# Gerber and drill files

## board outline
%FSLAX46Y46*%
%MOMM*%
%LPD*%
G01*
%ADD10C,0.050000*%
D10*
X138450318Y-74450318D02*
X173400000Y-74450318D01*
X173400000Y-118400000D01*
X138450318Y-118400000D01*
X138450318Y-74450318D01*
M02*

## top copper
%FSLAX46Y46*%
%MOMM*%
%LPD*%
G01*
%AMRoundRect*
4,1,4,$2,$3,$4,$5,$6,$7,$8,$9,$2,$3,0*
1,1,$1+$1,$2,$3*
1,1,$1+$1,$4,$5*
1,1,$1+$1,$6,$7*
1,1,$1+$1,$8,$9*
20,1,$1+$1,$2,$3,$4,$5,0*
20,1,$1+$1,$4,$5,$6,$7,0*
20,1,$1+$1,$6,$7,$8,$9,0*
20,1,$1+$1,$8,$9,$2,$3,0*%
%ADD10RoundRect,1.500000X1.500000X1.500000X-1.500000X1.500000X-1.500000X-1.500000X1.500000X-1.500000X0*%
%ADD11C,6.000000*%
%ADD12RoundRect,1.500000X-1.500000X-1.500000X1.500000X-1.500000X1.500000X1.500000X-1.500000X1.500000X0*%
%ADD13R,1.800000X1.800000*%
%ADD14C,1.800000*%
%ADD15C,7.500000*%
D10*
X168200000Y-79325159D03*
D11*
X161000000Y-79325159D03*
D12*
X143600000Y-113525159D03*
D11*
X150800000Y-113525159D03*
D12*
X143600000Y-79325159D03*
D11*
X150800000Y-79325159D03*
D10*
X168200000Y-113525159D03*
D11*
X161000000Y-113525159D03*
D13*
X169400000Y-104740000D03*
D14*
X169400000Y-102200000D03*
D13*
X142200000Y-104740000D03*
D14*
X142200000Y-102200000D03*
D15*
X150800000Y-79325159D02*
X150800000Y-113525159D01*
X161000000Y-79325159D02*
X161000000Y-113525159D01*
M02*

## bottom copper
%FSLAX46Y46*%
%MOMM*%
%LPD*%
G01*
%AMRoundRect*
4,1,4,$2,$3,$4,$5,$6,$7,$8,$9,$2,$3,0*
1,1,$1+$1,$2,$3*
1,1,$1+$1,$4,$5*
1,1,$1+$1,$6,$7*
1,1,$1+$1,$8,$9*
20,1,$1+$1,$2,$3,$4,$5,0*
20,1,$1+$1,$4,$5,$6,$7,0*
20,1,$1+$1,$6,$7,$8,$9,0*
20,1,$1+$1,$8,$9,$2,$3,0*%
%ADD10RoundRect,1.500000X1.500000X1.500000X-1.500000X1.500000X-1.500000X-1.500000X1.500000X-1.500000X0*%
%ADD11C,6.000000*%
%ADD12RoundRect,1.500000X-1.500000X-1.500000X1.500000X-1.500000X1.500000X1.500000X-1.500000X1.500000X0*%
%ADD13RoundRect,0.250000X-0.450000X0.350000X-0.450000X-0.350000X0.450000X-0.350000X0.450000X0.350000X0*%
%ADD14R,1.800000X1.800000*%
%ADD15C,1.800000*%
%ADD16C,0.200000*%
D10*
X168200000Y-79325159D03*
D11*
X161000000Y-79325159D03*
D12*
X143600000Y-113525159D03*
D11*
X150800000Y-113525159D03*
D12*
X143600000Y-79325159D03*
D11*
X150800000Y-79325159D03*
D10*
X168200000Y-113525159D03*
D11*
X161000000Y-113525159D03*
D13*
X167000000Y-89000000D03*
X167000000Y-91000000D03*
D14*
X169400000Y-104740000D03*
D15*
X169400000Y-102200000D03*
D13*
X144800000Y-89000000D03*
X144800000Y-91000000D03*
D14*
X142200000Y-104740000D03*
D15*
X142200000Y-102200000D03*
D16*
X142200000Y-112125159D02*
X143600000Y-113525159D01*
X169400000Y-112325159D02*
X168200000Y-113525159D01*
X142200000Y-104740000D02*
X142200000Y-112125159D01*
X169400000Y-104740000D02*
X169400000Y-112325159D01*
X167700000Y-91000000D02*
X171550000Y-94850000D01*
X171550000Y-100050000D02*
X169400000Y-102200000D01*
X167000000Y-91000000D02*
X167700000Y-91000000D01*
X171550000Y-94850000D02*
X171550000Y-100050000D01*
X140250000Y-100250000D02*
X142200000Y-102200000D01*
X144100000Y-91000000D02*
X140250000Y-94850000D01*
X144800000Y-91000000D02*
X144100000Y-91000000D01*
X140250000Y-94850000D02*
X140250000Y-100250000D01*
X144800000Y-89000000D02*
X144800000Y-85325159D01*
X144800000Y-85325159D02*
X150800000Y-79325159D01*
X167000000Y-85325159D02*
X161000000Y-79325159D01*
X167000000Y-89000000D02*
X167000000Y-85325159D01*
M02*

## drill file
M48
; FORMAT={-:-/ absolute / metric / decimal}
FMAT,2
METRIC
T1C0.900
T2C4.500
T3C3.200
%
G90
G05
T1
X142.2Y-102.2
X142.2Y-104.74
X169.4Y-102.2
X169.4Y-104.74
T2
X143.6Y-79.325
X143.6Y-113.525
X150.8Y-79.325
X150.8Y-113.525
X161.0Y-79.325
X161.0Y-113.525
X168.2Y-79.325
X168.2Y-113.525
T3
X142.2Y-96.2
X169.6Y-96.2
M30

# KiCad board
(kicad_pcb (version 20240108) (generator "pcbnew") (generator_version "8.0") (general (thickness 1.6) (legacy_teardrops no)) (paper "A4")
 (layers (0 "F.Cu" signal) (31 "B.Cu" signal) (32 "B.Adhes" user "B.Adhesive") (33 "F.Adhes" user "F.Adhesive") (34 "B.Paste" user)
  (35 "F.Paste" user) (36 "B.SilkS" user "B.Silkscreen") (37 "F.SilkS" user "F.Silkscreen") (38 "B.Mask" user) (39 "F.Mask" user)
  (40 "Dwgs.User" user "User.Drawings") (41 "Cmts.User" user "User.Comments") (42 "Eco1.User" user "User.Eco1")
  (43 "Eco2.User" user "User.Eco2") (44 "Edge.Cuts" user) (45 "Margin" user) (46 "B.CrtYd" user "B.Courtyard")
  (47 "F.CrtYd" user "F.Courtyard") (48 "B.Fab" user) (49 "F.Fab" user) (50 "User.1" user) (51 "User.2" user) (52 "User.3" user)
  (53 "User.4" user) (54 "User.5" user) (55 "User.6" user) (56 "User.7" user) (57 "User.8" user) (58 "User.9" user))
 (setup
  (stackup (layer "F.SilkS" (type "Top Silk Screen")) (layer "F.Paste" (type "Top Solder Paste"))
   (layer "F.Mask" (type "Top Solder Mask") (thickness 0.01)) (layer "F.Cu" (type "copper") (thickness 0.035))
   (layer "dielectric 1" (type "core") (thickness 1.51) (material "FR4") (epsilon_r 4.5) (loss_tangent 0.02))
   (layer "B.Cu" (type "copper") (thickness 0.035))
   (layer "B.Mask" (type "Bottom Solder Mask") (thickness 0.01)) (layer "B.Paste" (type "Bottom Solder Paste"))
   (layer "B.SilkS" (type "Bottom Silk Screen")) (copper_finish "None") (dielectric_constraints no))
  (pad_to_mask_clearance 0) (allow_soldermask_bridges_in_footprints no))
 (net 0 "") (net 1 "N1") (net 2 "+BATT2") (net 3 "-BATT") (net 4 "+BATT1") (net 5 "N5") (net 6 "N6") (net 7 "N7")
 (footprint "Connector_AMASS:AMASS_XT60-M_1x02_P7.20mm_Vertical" (layer "F.Cu") (at 168.2 79.325159 180)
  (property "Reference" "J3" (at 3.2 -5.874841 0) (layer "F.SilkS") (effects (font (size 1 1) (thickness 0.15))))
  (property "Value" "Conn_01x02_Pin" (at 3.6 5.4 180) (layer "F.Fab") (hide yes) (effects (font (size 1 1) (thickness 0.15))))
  (pad "1" thru_hole roundrect (at 0 0 180) (size 6 6) (drill 4.5) (layers "*.Cu" "*.Mask") (remove_unused_layers no)
   (roundrect_rratio 0.25) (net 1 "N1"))
  (pad "2" thru_hole circle (at 7.2 0 180) (size 6 6) (drill 4.5) (layers "*.Cu" "*.Mask") (remove_unused_layers no) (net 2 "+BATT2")))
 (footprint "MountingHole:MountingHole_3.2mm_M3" (layer "F.Cu") (at 169.6 96.2)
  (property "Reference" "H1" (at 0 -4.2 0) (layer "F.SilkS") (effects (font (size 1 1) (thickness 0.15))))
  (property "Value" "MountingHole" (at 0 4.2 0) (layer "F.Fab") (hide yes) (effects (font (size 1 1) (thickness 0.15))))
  (pad "" np_thru_hole circle (at 0 0) (size 3.2 3.2) (drill 3.2) (layers "*.Cu" "*.Mask")))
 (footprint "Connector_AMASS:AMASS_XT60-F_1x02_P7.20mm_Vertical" (layer "F.Cu") (at 143.6 113.525159)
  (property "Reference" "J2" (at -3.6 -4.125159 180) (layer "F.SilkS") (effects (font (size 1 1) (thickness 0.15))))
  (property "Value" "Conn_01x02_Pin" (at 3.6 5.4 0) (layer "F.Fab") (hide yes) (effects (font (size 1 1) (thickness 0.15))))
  (pad "1" thru_hole roundrect (at 0 0) (size 6 6) (drill 4.5) (layers "*.Cu" "*.Mask") (remove_unused_layers no) (roundrect_rratio 0.25)
   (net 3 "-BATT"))
  (pad "2" thru_hole circle (at 7.2 0) (size 6 6) (drill 4.5) (layers "*.Cu" "*.Mask") (remove_unused_layers no) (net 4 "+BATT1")))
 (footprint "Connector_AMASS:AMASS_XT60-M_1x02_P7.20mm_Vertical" (layer "F.Cu") (at 143.6 79.325159)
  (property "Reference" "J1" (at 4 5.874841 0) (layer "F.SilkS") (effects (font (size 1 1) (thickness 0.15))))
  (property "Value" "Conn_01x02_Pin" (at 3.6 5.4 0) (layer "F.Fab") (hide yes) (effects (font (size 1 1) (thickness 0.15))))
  (pad "1" thru_hole roundrect (at 0 0) (size 6 6) (drill 4.5) (layers "*.Cu" "*.Mask") (remove_unused_layers no) (roundrect_rratio 0.25)
   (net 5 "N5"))
  (pad "2" thru_hole circle (at 7.2 0) (size 6 6) (drill 4.5) (layers "*.Cu" "*.Mask") (remove_unused_layers no) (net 4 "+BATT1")))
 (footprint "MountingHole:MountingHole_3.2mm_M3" (layer "F.Cu") (at 142.2 96.2)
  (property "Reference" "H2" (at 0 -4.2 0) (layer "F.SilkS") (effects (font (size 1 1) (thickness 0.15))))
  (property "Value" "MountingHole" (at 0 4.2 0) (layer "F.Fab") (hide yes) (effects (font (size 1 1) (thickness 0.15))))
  (pad "" np_thru_hole circle (at 0 0) (size 3.2 3.2) (drill 3.2) (layers "*.Cu" "*.Mask")))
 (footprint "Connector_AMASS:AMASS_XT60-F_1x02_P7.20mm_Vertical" (layer "F.Cu") (at 168.2 113.525159 180)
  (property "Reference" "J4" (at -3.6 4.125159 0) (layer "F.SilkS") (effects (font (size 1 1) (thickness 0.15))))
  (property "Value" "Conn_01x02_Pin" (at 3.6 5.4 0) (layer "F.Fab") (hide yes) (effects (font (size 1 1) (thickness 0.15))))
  (pad "1" thru_hole roundrect (at 0 0 180) (size 6 6) (drill 4.5) (layers "*.Cu" "*.Mask") (remove_unused_layers no)
   (roundrect_rratio 0.25) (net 3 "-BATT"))
  (pad "2" thru_hole circle (at 7.2 0 180) (size 6 6) (drill 4.5) (layers "*.Cu" "*.Mask") (remove_unused_layers no) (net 2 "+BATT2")))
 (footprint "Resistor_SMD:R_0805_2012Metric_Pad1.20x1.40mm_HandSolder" (layer "B.Cu") (at 167 90 -90)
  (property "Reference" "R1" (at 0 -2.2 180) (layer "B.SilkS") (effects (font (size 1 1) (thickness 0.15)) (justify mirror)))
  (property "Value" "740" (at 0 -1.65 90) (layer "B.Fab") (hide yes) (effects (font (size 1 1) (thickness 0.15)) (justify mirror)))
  (pad "1" smd roundrect (at -1 0 270) (size 1.2 1.4) (layers "B.Cu" "B.Paste" "B.Mask") (roundrect_rratio 0.208333) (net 2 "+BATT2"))
  (pad "2" smd roundrect (at 1 0 270) (size 1.2 1.4) (layers "B.Cu" "B.Paste" "B.Mask") (roundrect_rratio 0.208333) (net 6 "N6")))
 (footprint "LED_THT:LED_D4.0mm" (layer "B.Cu") (at 169.4 104.74 90)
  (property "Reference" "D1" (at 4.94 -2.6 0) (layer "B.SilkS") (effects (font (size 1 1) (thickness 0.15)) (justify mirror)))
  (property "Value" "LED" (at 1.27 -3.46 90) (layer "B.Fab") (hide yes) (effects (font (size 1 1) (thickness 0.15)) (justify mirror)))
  (pad "1" thru_hole rect (at 0 0 90) (size 1.8 1.8) (drill 0.9) (layers "*.Cu" "*.Mask") (remove_unused_layers no) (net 3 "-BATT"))
  (pad "2" thru_hole circle (at 2.54 0 90) (size 1.8 1.8) (drill 0.9) (layers "*.Cu" "*.Mask") (remove_unused_layers no) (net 6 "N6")))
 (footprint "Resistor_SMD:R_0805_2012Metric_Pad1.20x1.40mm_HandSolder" (layer "B.Cu") (at 144.8 90 -90)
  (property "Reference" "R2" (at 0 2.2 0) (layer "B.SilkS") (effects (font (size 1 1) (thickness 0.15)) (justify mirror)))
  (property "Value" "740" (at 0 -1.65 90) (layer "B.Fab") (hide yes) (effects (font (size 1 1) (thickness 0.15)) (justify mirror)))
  (pad "1" smd roundrect (at -1 0 270) (size 1.2 1.4) (layers "B.Cu" "B.Paste" "B.Mask") (roundrect_rratio 0.208333) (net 4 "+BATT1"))
  (pad "2" smd roundrect (at 1 0 270) (size 1.2 1.4) (layers "B.Cu" "B.Paste" "B.Mask") (roundrect_rratio 0.208333) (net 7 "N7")))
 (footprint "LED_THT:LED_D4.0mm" (layer "B.Cu") (at 142.2 104.74 90)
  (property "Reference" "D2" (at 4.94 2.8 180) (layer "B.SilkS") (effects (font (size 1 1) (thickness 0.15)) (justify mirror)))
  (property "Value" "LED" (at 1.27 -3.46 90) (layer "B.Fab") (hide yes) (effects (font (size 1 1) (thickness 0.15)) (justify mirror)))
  (pad "1" thru_hole rect (at 0 0 90) (size 1.8 1.8) (drill 0.9) (layers "*.Cu" "*.Mask") (remove_unused_layers no) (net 3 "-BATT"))
  (pad "2" thru_hole circle (at 2.54 0 90) (size 1.8 1.8) (drill 0.9) (layers "*.Cu" "*.Mask") (remove_unused_layers no) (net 7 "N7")))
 (gr_rect (start 138.450318 74.450318) (end 173.4 118.4) (stroke (width 0.05) (type default)) (fill none) (layer "Edge.Cuts"))
 (segment (start 142.2 112.125159) (end 143.6 113.525159) (width 0.2) (layer "B.Cu") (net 3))
 (segment (start 169.4 112.325159) (end 168.2 113.525159) (width 0.2) (layer "B.Cu") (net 3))
 (segment (start 142.2 104.74) (end 142.2 112.125159) (width 0.2) (layer "B.Cu") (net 3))
 (segment (start 169.4 104.74) (end 169.4 112.325159) (width 0.2) (layer "B.Cu") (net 3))
 (segment (start 167.7 91) (end 171.55 94.85) (width 0.2) (layer "B.Cu") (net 6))
 (segment (start 171.55 100.05) (end 169.4 102.2) (width 0.2) (layer "B.Cu") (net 6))
 (segment (start 167 91) (end 167.7 91) (width 0.2) (layer "B.Cu") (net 6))
 (segment (start 171.55 94.85) (end 171.55 100.05) (width 0.2) (layer "B.Cu") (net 6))
 (segment (start 140.25 100.25) (end 142.2 102.2) (width 0.2) (layer "B.Cu") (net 7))
 (segment (start 144.1 91) (end 140.25 94.85) (width 0.2) (layer "B.Cu") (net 7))
 (segment (start 144.8 91) (end 144.1 91) (width 0.2) (layer "B.Cu") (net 7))
 (segment (start 140.25 94.85) (end 140.25 100.25) (width 0.2) (layer "B.Cu") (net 7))
 (segment (start 150.8 79.325159) (end 150.8 113.525159) (width 7.5) (layer "F.Cu") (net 4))
 (segment (start 144.8 89) (end 144.8 85.325159) (width 0.2) (layer "B.Cu") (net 4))
 (segment (start 144.8 85.325159) (end 150.8 79.325159) (width 0.2) (layer "B.Cu") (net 4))
 (segment (start 161 79.325159) (end 161 113.525159) (width 7.5) (layer "F.Cu") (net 2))
 (segment (start 167 85.325159) (end 161 79.325159) (width 0.2) (layer "B.Cu") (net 2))
 (segment (start 167 89) (end 167 85.325159) (width 0.2) (layer "B.Cu") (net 2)))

